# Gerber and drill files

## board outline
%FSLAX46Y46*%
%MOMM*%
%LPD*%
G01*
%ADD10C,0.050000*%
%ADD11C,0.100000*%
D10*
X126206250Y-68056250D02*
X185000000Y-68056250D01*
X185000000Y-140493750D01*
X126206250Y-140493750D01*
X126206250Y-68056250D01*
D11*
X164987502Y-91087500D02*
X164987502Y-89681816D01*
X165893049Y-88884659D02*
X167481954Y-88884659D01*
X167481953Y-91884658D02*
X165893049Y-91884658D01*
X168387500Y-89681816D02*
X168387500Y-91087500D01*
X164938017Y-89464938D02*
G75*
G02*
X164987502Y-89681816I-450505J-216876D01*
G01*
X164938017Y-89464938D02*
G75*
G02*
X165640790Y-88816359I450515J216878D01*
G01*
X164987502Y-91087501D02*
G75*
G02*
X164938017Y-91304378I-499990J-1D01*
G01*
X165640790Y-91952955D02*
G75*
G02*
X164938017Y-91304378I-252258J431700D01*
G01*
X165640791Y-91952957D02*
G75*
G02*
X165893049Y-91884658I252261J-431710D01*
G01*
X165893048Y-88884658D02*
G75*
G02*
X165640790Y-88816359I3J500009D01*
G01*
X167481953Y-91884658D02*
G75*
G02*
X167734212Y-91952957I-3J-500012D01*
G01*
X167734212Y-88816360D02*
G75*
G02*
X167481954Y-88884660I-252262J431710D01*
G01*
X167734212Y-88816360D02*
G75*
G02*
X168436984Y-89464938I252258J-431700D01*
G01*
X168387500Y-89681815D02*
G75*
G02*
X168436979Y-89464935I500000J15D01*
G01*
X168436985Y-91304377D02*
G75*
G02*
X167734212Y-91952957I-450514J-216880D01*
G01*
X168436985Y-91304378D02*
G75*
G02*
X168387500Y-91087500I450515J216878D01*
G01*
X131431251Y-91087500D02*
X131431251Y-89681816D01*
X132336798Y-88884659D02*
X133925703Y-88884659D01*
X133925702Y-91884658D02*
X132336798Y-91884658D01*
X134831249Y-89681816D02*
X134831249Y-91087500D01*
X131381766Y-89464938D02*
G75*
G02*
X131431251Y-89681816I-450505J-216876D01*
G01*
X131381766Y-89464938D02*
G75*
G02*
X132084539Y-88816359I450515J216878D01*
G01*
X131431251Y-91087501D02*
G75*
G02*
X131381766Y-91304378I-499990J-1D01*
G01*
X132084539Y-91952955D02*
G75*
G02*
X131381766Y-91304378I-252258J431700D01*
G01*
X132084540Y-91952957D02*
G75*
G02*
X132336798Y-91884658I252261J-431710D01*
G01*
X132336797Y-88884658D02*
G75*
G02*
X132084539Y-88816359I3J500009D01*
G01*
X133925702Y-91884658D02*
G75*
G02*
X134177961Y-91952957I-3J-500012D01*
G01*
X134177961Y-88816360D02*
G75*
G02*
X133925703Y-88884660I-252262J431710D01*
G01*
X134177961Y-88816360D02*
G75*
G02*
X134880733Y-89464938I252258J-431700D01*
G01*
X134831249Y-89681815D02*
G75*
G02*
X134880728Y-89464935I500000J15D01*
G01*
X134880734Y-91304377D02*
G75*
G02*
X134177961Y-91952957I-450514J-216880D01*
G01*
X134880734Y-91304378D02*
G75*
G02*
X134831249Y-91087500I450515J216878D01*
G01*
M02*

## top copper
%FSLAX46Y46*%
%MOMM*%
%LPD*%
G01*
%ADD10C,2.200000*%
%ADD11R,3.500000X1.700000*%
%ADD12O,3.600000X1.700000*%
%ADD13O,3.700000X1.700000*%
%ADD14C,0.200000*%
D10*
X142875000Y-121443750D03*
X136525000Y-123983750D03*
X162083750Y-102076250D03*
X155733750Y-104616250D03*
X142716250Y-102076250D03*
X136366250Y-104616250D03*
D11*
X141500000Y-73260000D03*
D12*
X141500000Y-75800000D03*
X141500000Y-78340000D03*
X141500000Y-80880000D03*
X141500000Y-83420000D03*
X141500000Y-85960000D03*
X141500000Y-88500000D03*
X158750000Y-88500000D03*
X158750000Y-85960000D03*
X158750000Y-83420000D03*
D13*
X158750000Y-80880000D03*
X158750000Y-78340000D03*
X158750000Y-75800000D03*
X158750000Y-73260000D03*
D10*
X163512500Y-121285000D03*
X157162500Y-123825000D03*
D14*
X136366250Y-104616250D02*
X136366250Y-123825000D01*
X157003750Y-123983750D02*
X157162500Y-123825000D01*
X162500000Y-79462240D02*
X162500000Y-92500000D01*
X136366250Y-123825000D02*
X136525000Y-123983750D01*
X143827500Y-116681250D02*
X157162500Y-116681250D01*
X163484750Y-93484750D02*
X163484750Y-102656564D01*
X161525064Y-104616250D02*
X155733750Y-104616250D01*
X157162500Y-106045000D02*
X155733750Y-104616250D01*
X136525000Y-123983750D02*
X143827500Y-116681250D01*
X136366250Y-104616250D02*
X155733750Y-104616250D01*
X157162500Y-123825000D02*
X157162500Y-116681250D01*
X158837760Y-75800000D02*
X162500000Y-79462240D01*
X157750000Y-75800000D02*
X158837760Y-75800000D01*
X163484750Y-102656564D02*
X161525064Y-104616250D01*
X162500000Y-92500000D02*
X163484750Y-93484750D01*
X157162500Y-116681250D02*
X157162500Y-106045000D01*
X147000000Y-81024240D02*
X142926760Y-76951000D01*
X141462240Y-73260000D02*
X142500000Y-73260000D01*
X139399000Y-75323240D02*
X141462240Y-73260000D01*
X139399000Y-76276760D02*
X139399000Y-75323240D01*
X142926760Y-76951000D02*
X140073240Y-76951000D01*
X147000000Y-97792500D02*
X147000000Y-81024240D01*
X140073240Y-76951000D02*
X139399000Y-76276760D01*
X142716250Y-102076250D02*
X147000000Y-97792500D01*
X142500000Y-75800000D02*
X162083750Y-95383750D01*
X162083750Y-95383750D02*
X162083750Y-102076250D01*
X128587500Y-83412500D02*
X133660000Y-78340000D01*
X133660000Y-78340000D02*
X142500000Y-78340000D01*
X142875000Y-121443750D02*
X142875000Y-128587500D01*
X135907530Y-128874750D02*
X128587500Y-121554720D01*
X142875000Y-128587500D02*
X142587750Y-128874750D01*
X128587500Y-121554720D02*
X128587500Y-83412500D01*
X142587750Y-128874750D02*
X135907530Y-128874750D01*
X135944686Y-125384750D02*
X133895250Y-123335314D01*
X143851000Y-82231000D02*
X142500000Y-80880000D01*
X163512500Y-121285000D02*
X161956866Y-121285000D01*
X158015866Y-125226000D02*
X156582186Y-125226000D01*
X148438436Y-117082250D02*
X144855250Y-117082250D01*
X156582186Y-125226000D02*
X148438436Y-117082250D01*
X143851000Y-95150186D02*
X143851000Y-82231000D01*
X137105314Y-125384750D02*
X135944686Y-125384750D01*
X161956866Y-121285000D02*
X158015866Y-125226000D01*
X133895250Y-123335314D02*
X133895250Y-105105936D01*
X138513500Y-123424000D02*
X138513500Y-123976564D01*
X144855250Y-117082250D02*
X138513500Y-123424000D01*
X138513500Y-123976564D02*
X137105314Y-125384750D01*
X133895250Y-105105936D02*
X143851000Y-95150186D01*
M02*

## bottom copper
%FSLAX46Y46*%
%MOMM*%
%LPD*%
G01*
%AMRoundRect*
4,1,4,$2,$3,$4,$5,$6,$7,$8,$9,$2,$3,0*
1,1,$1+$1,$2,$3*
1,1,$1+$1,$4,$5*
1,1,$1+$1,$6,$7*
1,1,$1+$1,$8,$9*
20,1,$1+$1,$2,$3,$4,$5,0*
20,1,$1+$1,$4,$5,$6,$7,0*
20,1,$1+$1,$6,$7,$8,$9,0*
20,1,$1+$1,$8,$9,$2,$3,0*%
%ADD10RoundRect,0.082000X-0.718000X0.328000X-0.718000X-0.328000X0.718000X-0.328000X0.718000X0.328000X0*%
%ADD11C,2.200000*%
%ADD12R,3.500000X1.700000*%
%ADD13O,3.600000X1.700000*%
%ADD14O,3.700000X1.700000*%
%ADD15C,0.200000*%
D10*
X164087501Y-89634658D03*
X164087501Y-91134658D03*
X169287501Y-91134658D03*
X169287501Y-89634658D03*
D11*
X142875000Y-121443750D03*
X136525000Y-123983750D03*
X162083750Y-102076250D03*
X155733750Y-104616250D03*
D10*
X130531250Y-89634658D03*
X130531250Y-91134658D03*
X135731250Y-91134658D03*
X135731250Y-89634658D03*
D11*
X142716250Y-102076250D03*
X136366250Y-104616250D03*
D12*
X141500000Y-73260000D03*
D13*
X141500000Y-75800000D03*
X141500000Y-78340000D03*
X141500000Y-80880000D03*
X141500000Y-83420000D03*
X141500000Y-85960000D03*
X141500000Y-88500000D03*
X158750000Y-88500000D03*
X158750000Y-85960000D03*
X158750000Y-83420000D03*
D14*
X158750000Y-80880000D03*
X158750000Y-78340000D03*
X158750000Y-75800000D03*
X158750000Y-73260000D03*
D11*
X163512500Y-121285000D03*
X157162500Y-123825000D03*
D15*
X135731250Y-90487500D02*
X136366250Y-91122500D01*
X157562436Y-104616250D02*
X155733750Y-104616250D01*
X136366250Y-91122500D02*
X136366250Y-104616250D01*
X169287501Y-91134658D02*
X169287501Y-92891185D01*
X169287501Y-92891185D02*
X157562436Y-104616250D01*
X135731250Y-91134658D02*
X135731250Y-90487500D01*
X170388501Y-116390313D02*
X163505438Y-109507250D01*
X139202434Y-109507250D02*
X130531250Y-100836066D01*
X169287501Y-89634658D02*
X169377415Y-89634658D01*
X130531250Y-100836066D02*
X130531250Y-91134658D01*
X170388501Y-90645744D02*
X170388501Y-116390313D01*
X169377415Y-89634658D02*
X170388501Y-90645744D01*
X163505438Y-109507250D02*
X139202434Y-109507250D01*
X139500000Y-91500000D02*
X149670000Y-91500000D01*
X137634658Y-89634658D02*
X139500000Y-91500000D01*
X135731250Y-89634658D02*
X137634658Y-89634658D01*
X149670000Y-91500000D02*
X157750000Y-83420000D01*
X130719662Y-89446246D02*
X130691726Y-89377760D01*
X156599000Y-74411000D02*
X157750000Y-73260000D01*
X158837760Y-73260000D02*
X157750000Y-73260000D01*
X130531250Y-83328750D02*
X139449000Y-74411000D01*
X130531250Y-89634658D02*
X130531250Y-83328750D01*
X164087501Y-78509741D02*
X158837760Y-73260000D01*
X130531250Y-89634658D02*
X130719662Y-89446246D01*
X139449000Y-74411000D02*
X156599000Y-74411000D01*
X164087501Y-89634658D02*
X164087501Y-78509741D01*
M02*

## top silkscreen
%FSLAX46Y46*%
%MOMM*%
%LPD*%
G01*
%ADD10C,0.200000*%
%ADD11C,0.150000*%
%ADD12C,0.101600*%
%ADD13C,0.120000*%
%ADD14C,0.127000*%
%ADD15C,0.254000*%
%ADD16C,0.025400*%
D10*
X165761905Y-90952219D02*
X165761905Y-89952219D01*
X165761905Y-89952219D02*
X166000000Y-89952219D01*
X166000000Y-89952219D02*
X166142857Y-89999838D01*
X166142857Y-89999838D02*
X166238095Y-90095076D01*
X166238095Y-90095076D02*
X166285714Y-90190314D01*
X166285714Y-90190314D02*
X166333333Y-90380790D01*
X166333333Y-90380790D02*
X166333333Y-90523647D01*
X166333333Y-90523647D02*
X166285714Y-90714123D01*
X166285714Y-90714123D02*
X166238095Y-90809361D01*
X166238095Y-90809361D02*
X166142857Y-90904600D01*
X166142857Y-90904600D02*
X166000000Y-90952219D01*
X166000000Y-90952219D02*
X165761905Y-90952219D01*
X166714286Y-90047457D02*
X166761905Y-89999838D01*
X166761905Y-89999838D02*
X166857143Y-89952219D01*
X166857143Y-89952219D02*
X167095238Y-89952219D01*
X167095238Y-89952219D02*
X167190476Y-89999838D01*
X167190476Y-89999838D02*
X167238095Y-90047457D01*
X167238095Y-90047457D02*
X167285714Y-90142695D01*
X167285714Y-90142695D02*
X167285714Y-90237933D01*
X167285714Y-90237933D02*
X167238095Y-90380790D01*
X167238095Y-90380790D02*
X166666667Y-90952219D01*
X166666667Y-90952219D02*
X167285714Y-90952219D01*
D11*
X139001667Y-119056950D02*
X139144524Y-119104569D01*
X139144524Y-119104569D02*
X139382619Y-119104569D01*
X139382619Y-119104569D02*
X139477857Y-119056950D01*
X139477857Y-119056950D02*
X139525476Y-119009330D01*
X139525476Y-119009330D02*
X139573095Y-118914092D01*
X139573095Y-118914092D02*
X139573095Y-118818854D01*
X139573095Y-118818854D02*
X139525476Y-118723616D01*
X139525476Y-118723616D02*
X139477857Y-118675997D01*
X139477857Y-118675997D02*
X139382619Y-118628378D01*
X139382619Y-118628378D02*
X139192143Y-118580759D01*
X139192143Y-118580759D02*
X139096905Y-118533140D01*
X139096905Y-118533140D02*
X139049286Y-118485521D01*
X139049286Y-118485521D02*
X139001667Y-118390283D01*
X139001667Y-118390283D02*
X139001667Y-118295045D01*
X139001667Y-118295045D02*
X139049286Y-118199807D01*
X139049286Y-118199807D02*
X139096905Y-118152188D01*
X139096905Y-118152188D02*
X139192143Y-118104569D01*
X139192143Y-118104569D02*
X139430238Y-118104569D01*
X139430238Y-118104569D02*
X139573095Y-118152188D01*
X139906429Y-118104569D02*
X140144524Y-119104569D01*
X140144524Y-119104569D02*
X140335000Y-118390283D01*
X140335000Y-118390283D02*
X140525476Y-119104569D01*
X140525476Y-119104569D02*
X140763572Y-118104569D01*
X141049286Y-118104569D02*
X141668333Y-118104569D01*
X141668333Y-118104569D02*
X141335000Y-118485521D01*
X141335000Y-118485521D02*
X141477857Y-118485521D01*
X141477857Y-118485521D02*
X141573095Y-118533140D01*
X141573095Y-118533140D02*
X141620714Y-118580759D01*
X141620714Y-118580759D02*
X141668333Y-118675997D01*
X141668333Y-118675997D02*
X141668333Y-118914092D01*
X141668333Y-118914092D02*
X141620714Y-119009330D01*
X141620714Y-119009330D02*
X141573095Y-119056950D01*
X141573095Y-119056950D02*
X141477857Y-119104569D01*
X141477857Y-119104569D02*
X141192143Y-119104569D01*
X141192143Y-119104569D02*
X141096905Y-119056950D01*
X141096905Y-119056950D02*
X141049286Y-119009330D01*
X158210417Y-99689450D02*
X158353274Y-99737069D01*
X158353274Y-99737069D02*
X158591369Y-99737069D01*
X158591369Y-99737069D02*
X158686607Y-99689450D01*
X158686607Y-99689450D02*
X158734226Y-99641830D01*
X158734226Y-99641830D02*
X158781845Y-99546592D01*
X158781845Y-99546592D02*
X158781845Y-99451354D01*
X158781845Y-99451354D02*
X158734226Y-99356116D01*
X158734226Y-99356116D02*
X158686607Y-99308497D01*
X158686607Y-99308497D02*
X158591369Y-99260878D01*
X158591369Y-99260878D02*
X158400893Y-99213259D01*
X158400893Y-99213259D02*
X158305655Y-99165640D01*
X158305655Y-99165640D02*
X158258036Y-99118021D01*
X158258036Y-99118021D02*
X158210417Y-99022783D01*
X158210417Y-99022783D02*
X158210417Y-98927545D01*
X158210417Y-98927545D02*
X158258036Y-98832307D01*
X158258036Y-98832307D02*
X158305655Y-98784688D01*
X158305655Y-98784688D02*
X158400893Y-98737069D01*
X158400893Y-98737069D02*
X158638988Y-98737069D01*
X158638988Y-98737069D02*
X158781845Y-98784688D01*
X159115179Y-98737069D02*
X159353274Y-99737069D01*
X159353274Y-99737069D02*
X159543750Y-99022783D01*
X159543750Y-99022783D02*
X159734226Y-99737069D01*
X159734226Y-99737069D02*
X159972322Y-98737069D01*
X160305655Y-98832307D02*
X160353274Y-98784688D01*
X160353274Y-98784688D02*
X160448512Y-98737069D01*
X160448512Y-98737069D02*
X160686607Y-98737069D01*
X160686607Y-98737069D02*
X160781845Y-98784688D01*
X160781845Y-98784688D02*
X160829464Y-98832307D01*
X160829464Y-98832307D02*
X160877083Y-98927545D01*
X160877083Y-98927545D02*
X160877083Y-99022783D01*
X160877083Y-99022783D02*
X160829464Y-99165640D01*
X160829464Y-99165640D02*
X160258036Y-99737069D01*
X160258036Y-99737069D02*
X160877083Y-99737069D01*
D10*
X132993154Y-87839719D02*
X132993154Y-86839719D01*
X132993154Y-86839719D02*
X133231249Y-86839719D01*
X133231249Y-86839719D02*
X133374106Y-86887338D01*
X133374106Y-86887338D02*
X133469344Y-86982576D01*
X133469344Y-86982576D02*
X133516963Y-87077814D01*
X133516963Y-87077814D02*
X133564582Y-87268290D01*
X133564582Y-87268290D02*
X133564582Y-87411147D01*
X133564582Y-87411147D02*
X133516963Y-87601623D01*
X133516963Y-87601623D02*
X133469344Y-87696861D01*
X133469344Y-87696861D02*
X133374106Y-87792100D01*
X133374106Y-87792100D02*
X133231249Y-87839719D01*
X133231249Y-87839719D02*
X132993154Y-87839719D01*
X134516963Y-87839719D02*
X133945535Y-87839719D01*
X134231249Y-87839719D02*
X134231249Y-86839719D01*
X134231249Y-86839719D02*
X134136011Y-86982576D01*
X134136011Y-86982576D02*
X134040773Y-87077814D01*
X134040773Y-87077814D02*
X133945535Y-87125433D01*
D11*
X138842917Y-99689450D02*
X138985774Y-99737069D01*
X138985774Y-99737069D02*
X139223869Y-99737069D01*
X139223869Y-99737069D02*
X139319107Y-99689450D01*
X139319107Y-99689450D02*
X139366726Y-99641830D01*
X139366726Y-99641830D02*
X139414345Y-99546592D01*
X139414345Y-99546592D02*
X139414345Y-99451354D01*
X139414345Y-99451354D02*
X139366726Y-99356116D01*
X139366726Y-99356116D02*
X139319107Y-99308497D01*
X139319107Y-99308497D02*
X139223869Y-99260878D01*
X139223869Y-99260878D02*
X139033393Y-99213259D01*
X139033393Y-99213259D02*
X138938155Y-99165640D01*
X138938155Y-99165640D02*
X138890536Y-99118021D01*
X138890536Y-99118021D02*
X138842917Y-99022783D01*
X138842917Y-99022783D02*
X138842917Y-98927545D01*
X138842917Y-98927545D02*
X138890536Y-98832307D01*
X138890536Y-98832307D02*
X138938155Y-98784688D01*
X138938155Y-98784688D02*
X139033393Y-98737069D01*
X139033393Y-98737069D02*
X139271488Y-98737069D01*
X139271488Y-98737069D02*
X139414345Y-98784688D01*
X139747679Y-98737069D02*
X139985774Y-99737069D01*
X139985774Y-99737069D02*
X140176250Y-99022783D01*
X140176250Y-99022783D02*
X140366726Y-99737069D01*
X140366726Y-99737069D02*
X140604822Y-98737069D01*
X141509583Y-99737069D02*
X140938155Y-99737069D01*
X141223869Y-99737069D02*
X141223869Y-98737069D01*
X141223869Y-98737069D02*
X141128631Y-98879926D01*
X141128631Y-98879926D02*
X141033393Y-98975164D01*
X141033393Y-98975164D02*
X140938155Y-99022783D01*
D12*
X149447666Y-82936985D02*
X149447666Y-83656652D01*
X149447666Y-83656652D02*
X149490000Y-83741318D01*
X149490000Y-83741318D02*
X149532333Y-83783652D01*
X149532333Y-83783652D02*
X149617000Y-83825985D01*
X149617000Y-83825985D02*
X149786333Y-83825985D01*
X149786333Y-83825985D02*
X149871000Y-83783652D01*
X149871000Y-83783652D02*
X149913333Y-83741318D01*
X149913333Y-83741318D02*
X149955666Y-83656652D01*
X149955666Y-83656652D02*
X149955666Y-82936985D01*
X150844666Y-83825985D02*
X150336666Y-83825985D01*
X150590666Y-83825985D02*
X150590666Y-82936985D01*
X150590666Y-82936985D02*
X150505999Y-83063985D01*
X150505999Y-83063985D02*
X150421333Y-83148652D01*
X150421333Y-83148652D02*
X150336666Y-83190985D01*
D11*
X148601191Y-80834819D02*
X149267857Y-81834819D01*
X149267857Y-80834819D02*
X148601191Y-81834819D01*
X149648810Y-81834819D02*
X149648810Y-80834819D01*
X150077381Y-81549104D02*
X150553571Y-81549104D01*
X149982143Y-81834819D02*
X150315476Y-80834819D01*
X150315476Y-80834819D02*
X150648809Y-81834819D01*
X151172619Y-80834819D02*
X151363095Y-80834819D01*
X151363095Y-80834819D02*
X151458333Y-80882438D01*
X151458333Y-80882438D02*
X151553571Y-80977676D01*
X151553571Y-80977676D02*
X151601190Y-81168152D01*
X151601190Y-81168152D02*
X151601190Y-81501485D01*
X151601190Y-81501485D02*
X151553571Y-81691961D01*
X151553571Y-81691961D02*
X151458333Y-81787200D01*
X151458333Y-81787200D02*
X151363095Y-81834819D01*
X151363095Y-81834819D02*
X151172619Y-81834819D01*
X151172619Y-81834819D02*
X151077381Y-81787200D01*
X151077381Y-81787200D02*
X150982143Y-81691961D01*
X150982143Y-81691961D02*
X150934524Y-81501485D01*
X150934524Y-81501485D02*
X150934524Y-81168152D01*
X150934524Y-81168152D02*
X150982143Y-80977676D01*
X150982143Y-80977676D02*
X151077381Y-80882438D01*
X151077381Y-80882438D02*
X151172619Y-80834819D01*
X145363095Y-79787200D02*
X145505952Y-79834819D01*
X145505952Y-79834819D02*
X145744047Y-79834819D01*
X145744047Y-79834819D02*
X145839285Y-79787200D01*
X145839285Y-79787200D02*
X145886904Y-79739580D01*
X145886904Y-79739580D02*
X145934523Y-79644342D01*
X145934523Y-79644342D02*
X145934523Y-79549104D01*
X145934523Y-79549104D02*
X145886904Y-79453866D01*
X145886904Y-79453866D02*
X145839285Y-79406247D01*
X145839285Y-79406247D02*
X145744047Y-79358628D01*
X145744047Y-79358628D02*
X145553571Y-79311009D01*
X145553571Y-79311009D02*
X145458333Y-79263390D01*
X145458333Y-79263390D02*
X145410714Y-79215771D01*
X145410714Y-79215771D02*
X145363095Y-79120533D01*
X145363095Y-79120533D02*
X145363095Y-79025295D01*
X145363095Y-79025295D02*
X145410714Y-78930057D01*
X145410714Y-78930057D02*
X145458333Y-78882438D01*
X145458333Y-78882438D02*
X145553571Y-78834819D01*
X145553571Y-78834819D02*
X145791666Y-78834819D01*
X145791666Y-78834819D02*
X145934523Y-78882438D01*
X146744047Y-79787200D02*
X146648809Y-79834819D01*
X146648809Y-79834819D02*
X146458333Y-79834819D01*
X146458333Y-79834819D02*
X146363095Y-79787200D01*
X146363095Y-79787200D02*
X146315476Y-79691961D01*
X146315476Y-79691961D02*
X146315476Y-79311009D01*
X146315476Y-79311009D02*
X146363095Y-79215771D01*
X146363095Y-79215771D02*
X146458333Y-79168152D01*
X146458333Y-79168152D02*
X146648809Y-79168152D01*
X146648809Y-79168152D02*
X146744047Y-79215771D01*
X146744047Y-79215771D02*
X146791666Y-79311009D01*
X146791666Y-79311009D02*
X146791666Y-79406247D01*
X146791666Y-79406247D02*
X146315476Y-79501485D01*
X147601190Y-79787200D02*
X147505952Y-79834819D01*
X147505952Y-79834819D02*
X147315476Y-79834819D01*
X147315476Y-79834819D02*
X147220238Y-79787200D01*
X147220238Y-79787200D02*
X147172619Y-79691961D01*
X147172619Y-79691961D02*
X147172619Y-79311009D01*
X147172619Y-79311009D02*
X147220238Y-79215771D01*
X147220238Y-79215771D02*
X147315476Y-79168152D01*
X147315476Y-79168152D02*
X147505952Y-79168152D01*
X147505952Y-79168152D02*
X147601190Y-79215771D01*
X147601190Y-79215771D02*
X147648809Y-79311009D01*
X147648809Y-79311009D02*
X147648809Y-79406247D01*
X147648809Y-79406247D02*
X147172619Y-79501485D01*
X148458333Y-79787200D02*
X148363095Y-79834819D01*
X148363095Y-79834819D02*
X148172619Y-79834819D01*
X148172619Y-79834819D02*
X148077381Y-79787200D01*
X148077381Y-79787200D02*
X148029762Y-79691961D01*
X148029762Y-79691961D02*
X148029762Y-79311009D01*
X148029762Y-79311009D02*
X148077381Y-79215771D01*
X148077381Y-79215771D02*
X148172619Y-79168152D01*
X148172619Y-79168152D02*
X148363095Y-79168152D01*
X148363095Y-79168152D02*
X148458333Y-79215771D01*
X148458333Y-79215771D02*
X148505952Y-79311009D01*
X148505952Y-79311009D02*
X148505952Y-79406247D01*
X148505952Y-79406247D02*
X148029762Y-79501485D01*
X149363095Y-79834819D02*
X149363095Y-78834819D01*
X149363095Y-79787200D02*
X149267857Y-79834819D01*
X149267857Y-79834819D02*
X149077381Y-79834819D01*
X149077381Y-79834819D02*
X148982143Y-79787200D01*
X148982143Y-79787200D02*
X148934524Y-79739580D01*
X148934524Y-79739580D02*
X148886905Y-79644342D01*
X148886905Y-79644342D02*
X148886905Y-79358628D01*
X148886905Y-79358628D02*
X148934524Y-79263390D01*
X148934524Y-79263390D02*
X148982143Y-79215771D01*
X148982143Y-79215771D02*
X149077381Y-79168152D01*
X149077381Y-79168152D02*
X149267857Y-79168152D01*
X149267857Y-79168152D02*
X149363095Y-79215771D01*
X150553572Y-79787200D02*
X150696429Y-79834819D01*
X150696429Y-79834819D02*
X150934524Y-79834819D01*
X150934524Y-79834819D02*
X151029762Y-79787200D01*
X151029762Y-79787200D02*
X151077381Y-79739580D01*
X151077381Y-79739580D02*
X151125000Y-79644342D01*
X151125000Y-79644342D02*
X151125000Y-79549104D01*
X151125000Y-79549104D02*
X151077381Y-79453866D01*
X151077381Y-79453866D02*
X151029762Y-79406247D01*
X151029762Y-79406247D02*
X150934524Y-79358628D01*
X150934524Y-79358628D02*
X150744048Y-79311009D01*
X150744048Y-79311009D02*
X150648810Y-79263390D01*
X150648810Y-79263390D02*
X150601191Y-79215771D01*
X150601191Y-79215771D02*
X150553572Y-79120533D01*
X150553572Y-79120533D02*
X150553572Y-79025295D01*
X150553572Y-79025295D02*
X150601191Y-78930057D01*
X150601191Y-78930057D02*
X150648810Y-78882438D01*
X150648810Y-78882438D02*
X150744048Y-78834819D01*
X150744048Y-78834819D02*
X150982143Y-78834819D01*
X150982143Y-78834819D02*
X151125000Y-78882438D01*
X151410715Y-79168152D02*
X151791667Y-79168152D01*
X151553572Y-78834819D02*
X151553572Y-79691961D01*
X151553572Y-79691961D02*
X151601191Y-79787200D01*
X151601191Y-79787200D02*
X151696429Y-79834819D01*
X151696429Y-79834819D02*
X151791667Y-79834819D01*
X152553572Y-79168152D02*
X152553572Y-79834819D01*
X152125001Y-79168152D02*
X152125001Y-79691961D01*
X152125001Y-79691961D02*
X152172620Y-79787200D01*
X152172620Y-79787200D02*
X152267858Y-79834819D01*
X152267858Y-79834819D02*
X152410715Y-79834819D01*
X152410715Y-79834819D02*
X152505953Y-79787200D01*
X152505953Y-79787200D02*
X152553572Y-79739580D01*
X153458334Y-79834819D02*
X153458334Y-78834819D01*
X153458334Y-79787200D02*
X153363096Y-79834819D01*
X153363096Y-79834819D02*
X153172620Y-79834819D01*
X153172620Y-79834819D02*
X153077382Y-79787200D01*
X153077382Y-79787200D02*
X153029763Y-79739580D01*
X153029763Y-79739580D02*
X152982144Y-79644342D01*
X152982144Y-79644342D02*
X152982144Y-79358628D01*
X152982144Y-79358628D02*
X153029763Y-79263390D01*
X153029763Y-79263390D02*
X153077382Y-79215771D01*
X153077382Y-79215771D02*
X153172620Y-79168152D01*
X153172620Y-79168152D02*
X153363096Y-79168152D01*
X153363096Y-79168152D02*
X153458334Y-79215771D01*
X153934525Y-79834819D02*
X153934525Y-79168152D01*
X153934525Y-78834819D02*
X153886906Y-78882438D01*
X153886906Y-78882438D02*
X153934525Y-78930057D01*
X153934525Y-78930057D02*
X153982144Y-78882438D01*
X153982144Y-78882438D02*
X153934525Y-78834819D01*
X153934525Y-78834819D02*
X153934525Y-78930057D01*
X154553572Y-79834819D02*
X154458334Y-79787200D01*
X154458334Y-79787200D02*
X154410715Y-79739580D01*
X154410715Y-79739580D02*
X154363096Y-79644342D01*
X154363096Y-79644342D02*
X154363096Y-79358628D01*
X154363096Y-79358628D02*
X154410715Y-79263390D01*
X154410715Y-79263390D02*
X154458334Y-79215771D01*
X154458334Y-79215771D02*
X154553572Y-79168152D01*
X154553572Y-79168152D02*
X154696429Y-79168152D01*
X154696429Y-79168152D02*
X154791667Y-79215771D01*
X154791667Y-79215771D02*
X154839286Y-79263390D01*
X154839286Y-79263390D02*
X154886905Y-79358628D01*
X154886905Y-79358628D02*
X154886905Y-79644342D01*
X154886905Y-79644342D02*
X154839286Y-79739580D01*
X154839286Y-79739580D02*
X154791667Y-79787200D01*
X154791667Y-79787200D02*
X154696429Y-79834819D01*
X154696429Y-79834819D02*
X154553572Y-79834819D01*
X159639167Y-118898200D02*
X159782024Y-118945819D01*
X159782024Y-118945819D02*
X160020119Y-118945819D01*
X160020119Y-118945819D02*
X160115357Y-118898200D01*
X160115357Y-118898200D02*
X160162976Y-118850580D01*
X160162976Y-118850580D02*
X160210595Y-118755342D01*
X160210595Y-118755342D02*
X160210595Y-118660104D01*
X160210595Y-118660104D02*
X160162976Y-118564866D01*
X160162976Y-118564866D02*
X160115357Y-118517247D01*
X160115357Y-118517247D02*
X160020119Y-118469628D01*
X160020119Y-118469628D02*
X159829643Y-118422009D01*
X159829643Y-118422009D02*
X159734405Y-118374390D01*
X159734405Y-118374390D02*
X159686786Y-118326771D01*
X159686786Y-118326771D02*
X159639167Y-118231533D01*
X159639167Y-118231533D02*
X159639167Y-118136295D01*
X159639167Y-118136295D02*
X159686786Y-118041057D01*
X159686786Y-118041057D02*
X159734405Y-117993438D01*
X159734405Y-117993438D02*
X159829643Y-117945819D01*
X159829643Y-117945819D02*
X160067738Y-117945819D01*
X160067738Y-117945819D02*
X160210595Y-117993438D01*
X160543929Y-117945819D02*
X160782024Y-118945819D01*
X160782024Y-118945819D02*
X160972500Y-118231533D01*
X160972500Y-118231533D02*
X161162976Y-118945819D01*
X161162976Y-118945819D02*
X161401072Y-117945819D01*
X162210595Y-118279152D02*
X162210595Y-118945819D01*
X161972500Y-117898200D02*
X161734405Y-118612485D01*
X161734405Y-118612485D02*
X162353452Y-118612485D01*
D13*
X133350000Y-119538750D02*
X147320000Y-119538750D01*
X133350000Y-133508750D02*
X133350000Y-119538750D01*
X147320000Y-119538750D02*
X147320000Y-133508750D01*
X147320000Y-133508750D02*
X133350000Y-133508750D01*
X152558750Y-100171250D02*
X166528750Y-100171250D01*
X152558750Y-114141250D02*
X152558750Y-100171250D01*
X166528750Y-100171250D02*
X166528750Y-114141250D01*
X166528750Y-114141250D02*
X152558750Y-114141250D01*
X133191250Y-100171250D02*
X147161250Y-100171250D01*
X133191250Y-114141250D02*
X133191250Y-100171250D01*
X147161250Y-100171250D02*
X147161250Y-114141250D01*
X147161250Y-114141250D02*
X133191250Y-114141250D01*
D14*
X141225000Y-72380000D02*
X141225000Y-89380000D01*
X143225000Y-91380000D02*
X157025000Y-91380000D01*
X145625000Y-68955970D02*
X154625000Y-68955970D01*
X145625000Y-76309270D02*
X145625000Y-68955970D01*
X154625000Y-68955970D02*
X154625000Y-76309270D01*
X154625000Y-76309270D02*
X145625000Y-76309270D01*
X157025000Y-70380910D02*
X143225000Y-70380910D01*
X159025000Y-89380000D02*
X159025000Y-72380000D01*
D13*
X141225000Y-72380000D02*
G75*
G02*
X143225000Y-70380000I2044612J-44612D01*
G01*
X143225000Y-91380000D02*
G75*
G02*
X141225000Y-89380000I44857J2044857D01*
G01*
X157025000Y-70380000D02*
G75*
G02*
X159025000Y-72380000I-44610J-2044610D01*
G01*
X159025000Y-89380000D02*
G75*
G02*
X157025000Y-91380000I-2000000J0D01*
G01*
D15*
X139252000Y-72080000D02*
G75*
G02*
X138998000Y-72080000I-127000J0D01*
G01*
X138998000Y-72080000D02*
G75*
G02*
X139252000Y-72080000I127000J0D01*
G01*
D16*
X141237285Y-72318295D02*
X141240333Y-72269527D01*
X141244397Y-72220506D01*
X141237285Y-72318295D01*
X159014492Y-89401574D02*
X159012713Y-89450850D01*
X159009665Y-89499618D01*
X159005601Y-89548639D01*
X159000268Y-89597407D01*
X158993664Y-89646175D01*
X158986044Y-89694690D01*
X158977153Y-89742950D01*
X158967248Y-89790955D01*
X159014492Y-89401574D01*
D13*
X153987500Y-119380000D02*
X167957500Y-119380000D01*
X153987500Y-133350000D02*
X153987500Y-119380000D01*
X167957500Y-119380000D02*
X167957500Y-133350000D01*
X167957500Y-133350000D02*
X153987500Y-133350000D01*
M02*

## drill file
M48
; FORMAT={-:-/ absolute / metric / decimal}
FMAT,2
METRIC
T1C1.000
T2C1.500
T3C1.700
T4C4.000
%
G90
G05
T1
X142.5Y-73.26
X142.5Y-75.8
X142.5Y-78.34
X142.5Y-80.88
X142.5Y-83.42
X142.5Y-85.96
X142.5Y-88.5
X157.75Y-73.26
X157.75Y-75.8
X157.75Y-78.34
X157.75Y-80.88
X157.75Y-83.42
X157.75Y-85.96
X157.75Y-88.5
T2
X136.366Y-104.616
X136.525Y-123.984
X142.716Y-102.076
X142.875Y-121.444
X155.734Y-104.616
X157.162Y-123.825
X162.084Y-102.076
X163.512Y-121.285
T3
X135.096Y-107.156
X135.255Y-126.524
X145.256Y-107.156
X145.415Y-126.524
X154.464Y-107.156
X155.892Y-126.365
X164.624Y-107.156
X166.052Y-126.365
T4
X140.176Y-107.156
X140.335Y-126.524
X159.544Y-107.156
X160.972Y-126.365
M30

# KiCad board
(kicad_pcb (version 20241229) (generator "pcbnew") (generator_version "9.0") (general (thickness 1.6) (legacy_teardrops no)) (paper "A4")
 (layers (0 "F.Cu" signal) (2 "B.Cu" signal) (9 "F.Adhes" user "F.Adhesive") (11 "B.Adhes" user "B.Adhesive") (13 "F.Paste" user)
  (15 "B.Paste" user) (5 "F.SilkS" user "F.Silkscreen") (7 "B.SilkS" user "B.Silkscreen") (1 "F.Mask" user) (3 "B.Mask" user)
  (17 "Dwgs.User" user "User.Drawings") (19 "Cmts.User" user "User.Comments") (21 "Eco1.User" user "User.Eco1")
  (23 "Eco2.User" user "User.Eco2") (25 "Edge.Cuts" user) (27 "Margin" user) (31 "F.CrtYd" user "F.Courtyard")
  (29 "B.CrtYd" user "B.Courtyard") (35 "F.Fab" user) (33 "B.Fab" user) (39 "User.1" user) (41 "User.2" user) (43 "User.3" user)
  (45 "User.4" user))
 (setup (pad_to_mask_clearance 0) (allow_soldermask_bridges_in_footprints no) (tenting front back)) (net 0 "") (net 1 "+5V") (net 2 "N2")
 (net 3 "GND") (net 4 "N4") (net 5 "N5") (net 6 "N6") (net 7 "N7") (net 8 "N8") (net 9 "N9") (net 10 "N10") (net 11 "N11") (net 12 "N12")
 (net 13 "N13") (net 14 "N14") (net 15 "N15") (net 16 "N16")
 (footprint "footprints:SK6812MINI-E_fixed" (layer "F.Cu") (at 166.6875 90.4875)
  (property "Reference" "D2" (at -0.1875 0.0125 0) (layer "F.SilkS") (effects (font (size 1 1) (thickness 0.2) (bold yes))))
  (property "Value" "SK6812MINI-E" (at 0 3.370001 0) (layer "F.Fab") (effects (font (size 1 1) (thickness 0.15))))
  (fp_line (start -1.699998 0.6) (end -1.699998 -0.805684) (stroke (width 0.1) (type solid)) (layer "Edge.Cuts"))
  (fp_line (start -0.794451 -1.602841) (end 0.794454 -1.602841) (stroke (width 0.1) (type solid)) (layer "Edge.Cuts"))
  (fp_line (start 0.794453 1.397158) (end -0.794451 1.397158) (stroke (width 0.1) (type solid)) (layer "Edge.Cuts"))
  (fp_line (start 1.7 -0.805684) (end 1.7 0.6) (stroke (width 0.1) (type solid)) (layer "Edge.Cuts"))
  (fp_arc (start -1.749483 -1.022562) (mid -1.712526 -0.91691) (end -1.699998 -0.805684) (stroke (width 0.1) (type solid))
   (layer "Edge.Cuts"))
  (fp_arc (start -1.749483 -1.022562) (mid -1.63807 -1.606877) (end -1.04671 -1.671141) (stroke (width 0.1) (type solid))
   (layer "Edge.Cuts"))
  (fp_arc (start -1.699998 0.600001) (mid -1.712526 0.711226) (end -1.749483 0.816878) (stroke (width 0.1) (type solid)) (layer "Edge.Cuts"))
  (fp_arc (start -1.04671 1.465455) (mid -1.638069 1.401192) (end -1.749483 0.816878) (stroke (width 0.1) (type solid)) (layer "Edge.Cuts"))
  (fp_arc (start -1.046709 1.465457) (mid -0.925121 1.414535) (end -0.794451 1.397158) (stroke (width 0.1) (type solid)) (layer "Edge.Cuts"))
  (fp_arc (start -0.794452 -1.602842) (mid -0.925122 -1.620219) (end -1.04671 -1.671141) (stroke (width 0.1) (type solid))
   (layer "Edge.Cuts"))
  (fp_arc (start 0.794453 1.397158) (mid 0.925124 1.414535) (end 1.046712 1.465457) (stroke (width 0.1) (type solid)) (layer "Edge.Cuts"))
  (fp_arc (start 1.046712 -1.67114) (mid 0.925124 -1.620218) (end 0.794454 -1.602841) (stroke (width 0.1) (type solid)) (layer "Edge.Cuts"))
  (fp_arc (start 1.046712 -1.67114) (mid 1.638072 -1.606876) (end 1.749485 -1.022562) (stroke (width 0.1) (type solid)) (layer "Edge.Cuts"))
  (fp_arc (start 1.7 -0.805685) (mid 1.712528 -0.91691) (end 1.749485 -1.022562) (stroke (width 0.1) (type solid)) (layer "Edge.Cuts"))
  (fp_arc (start 1.749485 0.816877) (mid 1.638073 1.401193) (end 1.046712 1.465457) (stroke (width 0.1) (type solid)) (layer "Edge.Cuts"))
  (fp_arc (start 1.749485 0.816878) (mid 1.712528 0.711226) (end 1.7 0.6) (stroke (width 0.1) (type solid)) (layer "Edge.Cuts"))
  (pad "1" smd roundrect (at -2.599999 -0.852842 270) (size 0.82 1.6) (layers "B.Cu" "B.Mask" "B.Paste") (roundrect_rratio 0.1)
   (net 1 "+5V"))
  (pad "2" smd roundrect (at -2.599999 0.647158 270) (size 0.82 1.6) (layers "B.Cu" "B.Mask" "B.Paste") (roundrect_rratio 0.1) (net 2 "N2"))
  (pad "3" smd roundrect (at 2.600001 0.647158 270) (size 0.82 1.6) (layers "B.Cu" "B.Mask" "B.Paste") (roundrect_rratio 0.1) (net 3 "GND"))
  (pad "4" smd roundrect (at 2.600001 -0.852842 270) (size 0.82 1.6) (layers "B.Cu" "B.Mask" "B.Paste") (roundrect_rratio 0.1) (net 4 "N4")))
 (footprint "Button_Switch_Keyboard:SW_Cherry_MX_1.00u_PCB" (layer "F.Cu") (at 142.82 117.03875)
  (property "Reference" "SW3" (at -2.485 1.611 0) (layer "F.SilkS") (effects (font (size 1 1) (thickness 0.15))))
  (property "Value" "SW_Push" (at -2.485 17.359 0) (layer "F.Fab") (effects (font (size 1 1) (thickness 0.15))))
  (fp_line (start -9.47 2.5) (end 4.5 2.5) (stroke (width 0.12) (type solid)) (layer "F.SilkS"))
  (fp_line (start -9.47 16.47) (end -9.47 2.5) (stroke (width 0.12) (type solid)) (layer "F.SilkS"))
  (fp_line (start 4.5 2.5) (end 4.5 16.47) (stroke (width 0.12) (type solid)) (layer "F.SilkS"))
  (fp_line (start 4.5 16.47) (end -9.47 16.47) (stroke (width 0.12) (type solid)) (layer "F.SilkS"))
  (pad "" np_thru_hole circle (at -7.565 9.485) (size 1.7 1.7) (drill 1.7) (layers "*.Cu" "*.Mask"))
  (pad "" np_thru_hole circle (at -2.485 9.485) (size 4 4) (drill 4) (layers "*.Cu" "*.Mask"))
  (pad "" np_thru_hole circle (at 2.595 9.485) (size 1.7 1.7) (drill 1.7) (layers "*.Cu" "*.Mask"))
  (pad "1" thru_hole circle (at 0.055 4.405) (size 2.2 2.2) (drill 1.5) (layers "*.Cu" "*.Mask") (remove_unused_layers no) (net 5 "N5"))
  (pad "2" thru_hole circle (at -6.295 6.945) (size 2.2 2.2) (drill 1.5) (layers "*.Cu" "*.Mask") (remove_unused_layers no) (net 3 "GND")))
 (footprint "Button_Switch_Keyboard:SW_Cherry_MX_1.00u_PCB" (layer "F.Cu") (at 162.02875 97.67125)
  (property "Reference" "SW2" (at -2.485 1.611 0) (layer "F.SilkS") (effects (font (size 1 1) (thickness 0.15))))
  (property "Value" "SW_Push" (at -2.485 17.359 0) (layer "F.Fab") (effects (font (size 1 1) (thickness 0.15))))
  (fp_line (start -9.47 2.5) (end 4.5 2.5) (stroke (width 0.12) (type solid)) (layer "F.SilkS"))
  (fp_line (start -9.47 16.47) (end -9.47 2.5) (stroke (width 0.12) (type solid)) (layer "F.SilkS"))
  (fp_line (start 4.5 2.5) (end 4.5 16.47) (stroke (width 0.12) (type solid)) (layer "F.SilkS"))
  (fp_line (start 4.5 16.47) (end -9.47 16.47) (stroke (width 0.12) (type solid)) (layer "F.SilkS"))
  (pad "" np_thru_hole circle (at -7.565 9.485) (size 1.7 1.7) (drill 1.7) (layers "*.Cu" "*.Mask"))
  (pad "" np_thru_hole circle (at -2.485 9.485) (size 4 4) (drill 4) (layers "*.Cu" "*.Mask"))
  (pad "" np_thru_hole circle (at 2.595 9.485) (size 1.7 1.7) (drill 1.7) (layers "*.Cu" "*.Mask"))
  (pad "1" thru_hole circle (at 0.055 4.405) (size 2.2 2.2) (drill 1.5) (layers "*.Cu" "*.Mask") (remove_unused_layers no) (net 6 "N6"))
  (pad "2" thru_hole circle (at -6.295 6.945) (size 2.2 2.2) (drill 1.5) (layers "*.Cu" "*.Mask") (remove_unused_layers no) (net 3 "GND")))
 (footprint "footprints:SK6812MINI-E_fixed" (layer "F.Cu") (at 133.131249 90.4875)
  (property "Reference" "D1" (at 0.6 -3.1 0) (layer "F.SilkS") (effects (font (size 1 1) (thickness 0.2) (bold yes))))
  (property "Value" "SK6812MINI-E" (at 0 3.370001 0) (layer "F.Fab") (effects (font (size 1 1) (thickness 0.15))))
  (fp_line (start -1.699998 0.6) (end -1.699998 -0.805684) (stroke (width 0.1) (type solid)) (layer "Edge.Cuts"))
  (fp_line (start -0.794451 -1.602841) (end 0.794454 -1.602841) (stroke (width 0.1) (type solid)) (layer "Edge.Cuts"))
  (fp_line (start 0.794453 1.397158) (end -0.794451 1.397158) (stroke (width 0.1) (type solid)) (layer "Edge.Cuts"))
  (fp_line (start 1.7 -0.805684) (end 1.7 0.6) (stroke (width 0.1) (type solid)) (layer "Edge.Cuts"))
  (fp_arc (start -1.749483 -1.022562) (mid -1.712526 -0.91691) (end -1.699998 -0.805684) (stroke (width 0.1) (type solid))
   (layer "Edge.Cuts"))
  (fp_arc (start -1.749483 -1.022562) (mid -1.63807 -1.606877) (end -1.04671 -1.671141) (stroke (width 0.1) (type solid))
   (layer "Edge.Cuts"))
  (fp_arc (start -1.699998 0.600001) (mid -1.712526 0.711226) (end -1.749483 0.816878) (stroke (width 0.1) (type solid)) (layer "Edge.Cuts"))
  (fp_arc (start -1.04671 1.465455) (mid -1.638069 1.401192) (end -1.749483 0.816878) (stroke (width 0.1) (type solid)) (layer "Edge.Cuts"))
  (fp_arc (start -1.046709 1.465457) (mid -0.925121 1.414535) (end -0.794451 1.397158) (stroke (width 0.1) (type solid)) (layer "Edge.Cuts"))
  (fp_arc (start -0.794452 -1.602842) (mid -0.925122 -1.620219) (end -1.04671 -1.671141) (stroke (width 0.1) (type solid))
   (layer "Edge.Cuts"))
  (fp_arc (start 0.794453 1.397158) (mid 0.925124 1.414535) (end 1.046712 1.465457) (stroke (width 0.1) (type solid)) (layer "Edge.Cuts"))
  (fp_arc (start 1.046712 -1.67114) (mid 0.925124 -1.620218) (end 0.794454 -1.602841) (stroke (width 0.1) (type solid)) (layer "Edge.Cuts"))
  (fp_arc (start 1.046712 -1.67114) (mid 1.638072 -1.606876) (end 1.749485 -1.022562) (stroke (width 0.1) (type solid)) (layer "Edge.Cuts"))
  (fp_arc (start 1.7 -0.805685) (mid 1.712528 -0.91691) (end 1.749485 -1.022562) (stroke (width 0.1) (type solid)) (layer "Edge.Cuts"))
  (fp_arc (start 1.749485 0.816877) (mid 1.638073 1.401193) (end 1.046712 1.465457) (stroke (width 0.1) (type solid)) (layer "Edge.Cuts"))
  (fp_arc (start 1.749485 0.816878) (mid 1.712528 0.711226) (end 1.7 0.6) (stroke (width 0.1) (type solid)) (layer "Edge.Cuts"))
  (pad "1" smd roundrect (at -2.599999 -0.852842 270) (size 0.82 1.6) (layers "B.Cu" "B.Mask" "B.Paste") (roundrect_rratio 0.1)
   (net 1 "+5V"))
  (pad "2" smd roundrect (at -2.599999 0.647158 270) (size 0.82 1.6) (layers "B.Cu" "B.Mask" "B.Paste") (roundrect_rratio 0.1) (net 4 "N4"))
  (pad "3" smd roundrect (at 2.600001 0.647158 270) (size 0.82 1.6) (layers "B.Cu" "B.Mask" "B.Paste") (roundrect_rratio 0.1) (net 3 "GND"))
  (pad "4" smd roundrect (at 2.600001 -0.852842 270) (size 0.82 1.6) (layers "B.Cu" "B.Mask" "B.Paste") (roundrect_rratio 0.1) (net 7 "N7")))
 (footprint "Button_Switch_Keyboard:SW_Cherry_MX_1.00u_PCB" (layer "F.Cu") (at 142.66125 97.67125)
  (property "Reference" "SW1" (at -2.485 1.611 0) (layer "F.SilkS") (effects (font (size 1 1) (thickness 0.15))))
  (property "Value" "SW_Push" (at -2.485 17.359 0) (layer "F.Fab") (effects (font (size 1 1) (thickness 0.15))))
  (fp_line (start -9.47 2.5) (end 4.5 2.5) (stroke (width 0.12) (type solid)) (layer "F.SilkS"))
  (fp_line (start -9.47 16.47) (end -9.47 2.5) (stroke (width 0.12) (type solid)) (layer "F.SilkS"))
  (fp_line (start 4.5 2.5) (end 4.5 16.47) (stroke (width 0.12) (type solid)) (layer "F.SilkS"))
  (fp_line (start 4.5 16.47) (end -9.47 16.47) (stroke (width 0.12) (type solid)) (layer "F.SilkS"))
  (pad "" np_thru_hole circle (at -7.565 9.485) (size 1.7 1.7) (drill 1.7) (layers "*.Cu" "*.Mask"))
  (pad "" np_thru_hole circle (at -2.485 9.485) (size 4 4) (drill 4) (layers "*.Cu" "*.Mask"))
  (pad "" np_thru_hole circle (at 2.595 9.485) (size 1.7 1.7) (drill 1.7) (layers "*.Cu" "*.Mask"))
  (pad "1" thru_hole circle (at 0.055 4.405) (size 2.2 2.2) (drill 1.5) (layers "*.Cu" "*.Mask") (remove_unused_layers no) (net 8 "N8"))
  (pad "2" thru_hole circle (at -6.295 6.945) (size 2.2 2.2) (drill 1.5) (layers "*.Cu" "*.Mask") (remove_unused_layers no) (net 3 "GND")))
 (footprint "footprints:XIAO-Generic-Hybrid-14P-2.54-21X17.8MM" (layer "F.Cu") (at 150.125 80.88)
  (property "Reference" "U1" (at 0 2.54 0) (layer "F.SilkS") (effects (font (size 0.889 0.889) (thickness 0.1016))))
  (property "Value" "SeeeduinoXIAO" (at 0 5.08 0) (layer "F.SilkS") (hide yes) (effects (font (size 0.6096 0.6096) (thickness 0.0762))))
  (fp_line (start -8.9 -8.5) (end -8.9 8.5) (stroke (width 0.127) (type solid)) (layer "F.SilkS"))
  (fp_line (start -6.9 10.5) (end 6.9 10.5) (stroke (width 0.127) (type solid)) (layer "F.SilkS"))
  (fp_line (start -4.5 -11.92403) (end 4.5 -11.92403) (stroke (width 0.127) (type solid)) (layer "F.SilkS"))
  (fp_line (start -4.5 -4.57073) (end -4.5 -11.92403) (stroke (width 0.127) (type solid)) (layer "F.SilkS"))
  (fp_line (start 4.5 -11.92403) (end 4.5 -4.57073) (stroke (width 0.127) (type solid)) (layer "F.SilkS"))
  (fp_line (start 4.5 -4.57073) (end -4.5 -4.57073) (stroke (width 0.127) (type solid)) (layer "F.SilkS"))
  (fp_line (start 6.9 -10.49909) (end -6.9 -10.49909) (stroke (width 0.127) (type solid)) (layer "F.SilkS"))
  (fp_line (start 8.9 8.5) (end 8.9 -8.5) (stroke (width 0.127) (type solid)) (layer "F.SilkS"))
  (fp_arc (start -8.9 -8.5) (mid -8.301491 -9.901491) (end -6.9 -10.5) (stroke (width 0.12) (type solid)) (layer "F.SilkS"))
  (fp_arc (start -6.9 10.5) (mid -8.301423 9.901423) (end -8.9 8.5) (stroke (width 0.12) (type solid)) (layer "F.SilkS"))
  (fp_arc (start 6.9 -10.5) (mid 8.301491 -9.901491) (end 8.9 -8.5) (stroke (width 0.12) (type solid)) (layer "F.SilkS"))
  (fp_arc (start 8.9 8.5) (mid 8.314214 9.914214) (end 6.9 10.5) (stroke (width 0.12) (type solid)) (layer "F.SilkS"))
  (fp_circle (center -11 -8.8) (end -11 -9.054) (stroke (width 0) (type solid)) (fill yes) (layer "F.SilkS"))
  (fp_poly
   (pts (xy -8.887715 -8.561705) (xy -8.884667 -8.610473) (xy -8.880603 -8.659494)) (stroke (width 0.0254) (type solid)) (fill no)
   (layer "F.SilkS"))
  (fp_poly
   (pts (xy 8.889492 8.521574) (xy 8.887713 8.57085) (xy 8.884665 8.619618) (xy 8.880601 8.668639) (xy 8.875268 8.717407)
    (xy 8.868664 8.766175) (xy 8.861044 8.81469) (xy 8.852153 8.86295) (xy 8.842248 8.910955))
   (stroke (width 0.0254) (type solid)) (fill no) (layer "F.SilkS"))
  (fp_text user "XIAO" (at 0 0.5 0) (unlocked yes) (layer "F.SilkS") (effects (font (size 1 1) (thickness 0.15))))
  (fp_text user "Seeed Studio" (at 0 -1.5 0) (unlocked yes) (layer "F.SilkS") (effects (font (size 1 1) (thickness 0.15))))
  (pad "1" thru_hole rect (at -7.625 -7.62) (size 3.5 1.7) (drill 1 (offset -1 0)) (layers "*.Cu" "*.Mask") (remove_unused_layers no)
   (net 8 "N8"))
  (pad "2" thru_hole oval (at -7.625 -5.08) (size 3.6 1.7) (drill 1 (offset -1 0)) (layers "*.Cu" "*.Mask") (remove_unused_layers no)
   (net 6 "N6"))
  (pad "3" thru_hole oval (at -7.625 -2.54) (size 3.6 1.7) (drill 1 (offset -1 0)) (layers "*.Cu" "*.Mask") (remove_unused_layers no)
   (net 5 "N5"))
  (pad "4" thru_hole oval (at -7.625 0) (size 3.6 1.7) (drill 1 (offset -1 0)) (layers "*.Cu" "*.Mask") (remove_unused_layers no)
   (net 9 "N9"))
  (pad "5" thru_hole oval (at -7.625 2.54) (size 3.6 1.7) (drill 1 (offset -1 0)) (layers "*.Cu" "*.Mask") (remove_unused_layers no)
   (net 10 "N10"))
  (pad "6" thru_hole oval (at -7.625 5.08 180) (size 3.6 1.7) (drill 1 (offset 1 0)) (layers "*.Cu" "*.Mask") (remove_unused_layers no)
   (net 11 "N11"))
  (pad "7" thru_hole oval (at -7.625 7.62) (size 3.6 1.7) (drill 1 (offset -1 0)) (layers "*.Cu" "*.Mask") (remove_unused_layers no)
   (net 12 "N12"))
  (pad "8" thru_hole oval (at 7.625 7.62) (size 3.6 1.7) (drill 1 (offset 1 0)) (layers "*.Cu" "*.Mask") (remove_unused_layers no)
   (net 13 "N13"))
  (pad "9" thru_hole oval (at 7.625 5.08) (size 3.6 1.7) (drill 1 (offset 1 0)) (layers "*.Cu" "*.Mask") (remove_unused_layers no)
   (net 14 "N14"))
  (pad "10" thru_hole oval (at 7.625 2.54) (size 3.6 1.7) (drill 1 (offset 1 0)) (layers "*.Cu" "*.Mask") (remove_unused_layers no)
   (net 7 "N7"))
  (pad "11" thru_hole oval (at 7.625 0) (size 3.7 1.7) (drill 1 (offset 1 0)) (layers "*.Cu" "*.Mask") (remove_unused_layers no)
   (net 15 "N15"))
  (pad "12" thru_hole oval (at 7.625 -2.54) (size 3.7 1.7) (drill 1 (offset 1 0)) (layers "*.Cu" "*.Mask") (remove_unused_layers no)
   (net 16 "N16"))
  (pad "13" thru_hole oval (at 7.625 -5.08) (size 3.7 1.7) (drill 1 (offset 1 0)) (layers "*.Cu" "*.Mask") (remove_unused_layers no)
   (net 3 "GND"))
  (pad "14" thru_hole oval (at 7.625 -7.62) (size 3.7 1.7) (drill 1 (offset 1 0)) (layers "*.Cu" "*.Mask") (remove_unused_layers no)
   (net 1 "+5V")))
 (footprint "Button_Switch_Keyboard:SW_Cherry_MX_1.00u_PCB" (layer "F.Cu") (at 163.4575 116.88)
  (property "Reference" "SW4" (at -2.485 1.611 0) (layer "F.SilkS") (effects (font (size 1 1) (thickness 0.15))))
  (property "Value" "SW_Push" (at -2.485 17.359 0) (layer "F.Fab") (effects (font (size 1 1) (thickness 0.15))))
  (fp_line (start -9.47 2.5) (end 4.5 2.5) (stroke (width 0.12) (type solid)) (layer "F.SilkS"))
  (fp_line (start -9.47 16.47) (end -9.47 2.5) (stroke (width 0.12) (type solid)) (layer "F.SilkS"))
  (fp_line (start 4.5 2.5) (end 4.5 16.47) (stroke (width 0.12) (type solid)) (layer "F.SilkS"))
  (fp_line (start 4.5 16.47) (end -9.47 16.47) (stroke (width 0.12) (type solid)) (layer "F.SilkS"))
  (pad "" np_thru_hole circle (at -7.565 9.485) (size 1.7 1.7) (drill 1.7) (layers "*.Cu" "*.Mask"))
  (pad "" np_thru_hole circle (at -2.485 9.485) (size 4 4) (drill 4) (layers "*.Cu" "*.Mask"))
  (pad "" np_thru_hole circle (at 2.595 9.485) (size 1.7 1.7) (drill 1.7) (layers "*.Cu" "*.Mask"))
  (pad "1" thru_hole circle (at 0.055 4.405) (size 2.2 2.2) (drill 1.5) (layers "*.Cu" "*.Mask") (remove_unused_layers no) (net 9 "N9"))
  (pad "2" thru_hole circle (at -6.295 6.945) (size 2.2 2.2) (drill 1.5) (layers "*.Cu" "*.Mask") (remove_unused_layers no) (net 3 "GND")))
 (gr_rect (start 126.20625 68.05625) (end 185 140.49375) (stroke (width 0.05) (type solid)) (fill no) (layer "Edge.Cuts"))
 (segment (start 136.36625 104.61625) (end 136.36625 123.825) (width 0.2) (layer "F.Cu") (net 3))
 (segment (start 157.00375 123.98375) (end 157.1625 123.825) (width 0.2) (layer "F.Cu") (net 3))
 (segment (start 162.5 79.46224) (end 162.5 92.5) (width 0.2) (layer "F.Cu") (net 3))
 (segment (start 136.36625 123.825) (end 136.525 123.98375) (width 0.2) (layer "F.Cu") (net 3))
 (segment (start 143.8275 116.68125) (end 157.1625 116.68125) (width 0.2) (layer "F.Cu") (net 3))
 (segment (start 163.48475 93.48475) (end 163.48475 102.656564) (width 0.2) (layer "F.Cu") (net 3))
 (segment (start 161.525064 104.61625) (end 155.73375 104.61625) (width 0.2) (layer "F.Cu") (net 3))
 (segment (start 157.1625 106.045) (end 155.73375 104.61625) (width 0.2) (layer "F.Cu") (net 3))
 (segment (start 136.525 123.98375) (end 143.8275 116.68125) (width 0.2) (layer "F.Cu") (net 3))
 (segment (start 136.36625 104.61625) (end 155.73375 104.61625) (width 0.2) (layer "F.Cu") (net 3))
 (segment (start 157.1625 123.825) (end 157.1625 116.68125) (width 0.2) (layer "F.Cu") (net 3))
 (segment (start 158.83776 75.8) (end 162.5 79.46224) (width 0.2) (layer "F.Cu") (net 3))
 (segment (start 157.75 75.8) (end 158.83776 75.8) (width 0.2) (layer "F.Cu") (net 3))
 (segment (start 163.48475 102.656564) (end 161.525064 104.61625) (width 0.2) (layer "F.Cu") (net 3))
 (segment (start 162.5 92.5) (end 163.48475 93.48475) (width 0.2) (layer "F.Cu") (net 3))
 (segment (start 157.1625 116.68125) (end 157.1625 106.045) (width 0.2) (layer "F.Cu") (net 3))
 (segment (start 135.73125 90.4875) (end 136.36625 91.1225) (width 0.2) (layer "B.Cu") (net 3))
 (segment (start 157.562436 104.61625) (end 155.73375 104.61625) (width 0.2) (layer "B.Cu") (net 3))
 (segment (start 136.36625 91.1225) (end 136.36625 104.61625) (width 0.2) (layer "B.Cu") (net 3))
 (segment (start 169.287501 91.134658) (end 169.287501 92.891185) (width 0.2) (layer "B.Cu") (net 3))
 (segment (start 169.287501 92.891185) (end 157.562436 104.61625) (width 0.2) (layer "B.Cu") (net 3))
 (segment (start 135.73125 91.134658) (end 135.73125 90.4875) (width 0.2) (layer "B.Cu") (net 3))
 (segment (start 170.388501 116.390313) (end 163.505438 109.50725) (width 0.2) (layer "B.Cu") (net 4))
 (segment (start 139.202434 109.50725) (end 130.53125 100.836066) (width 0.2) (layer "B.Cu") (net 4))
 (segment (start 169.287501 89.634658) (end 169.377415 89.634658) (width 0.2) (layer "B.Cu") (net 4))
 (segment (start 130.53125 100.836066) (end 130.53125 91.134658) (width 0.2) (layer "B.Cu") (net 4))
 (segment (start 170.388501 90.645744) (end 170.388501 116.390313) (width 0.2) (layer "B.Cu") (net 4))
 (segment (start 169.377415 89.634658) (end 170.388501 90.645744) (width 0.2) (layer "B.Cu") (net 4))
 (segment (start 163.505438 109.50725) (end 139.202434 109.50725) (width 0.2) (layer "B.Cu") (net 4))
 (segment (start 139.5 91.5) (end 149.67 91.5) (width 0.2) (layer "B.Cu") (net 7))
 (segment (start 137.634658 89.634658) (end 139.5 91.5) (width 0.2) (layer "B.Cu") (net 7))
 (segment (start 135.73125 89.634658) (end 137.634658 89.634658) (width 0.2) (layer "B.Cu") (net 7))
 (segment (start 149.67 91.5) (end 157.75 83.42) (width 0.2) (layer "B.Cu") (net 7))
 (segment (start 130.719662 89.446246) (end 130.691726 89.37776) (width 0.2) (layer "B.Cu") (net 1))
 (segment (start 156.599 74.411) (end 157.75 73.26) (width 0.2) (layer "B.Cu") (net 1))
 (segment (start 158.83776 73.26) (end 157.75 73.26) (width 0.2) (layer "B.Cu") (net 1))
 (segment (start 130.53125 83.32875) (end 139.449 74.411) (width 0.2) (layer "B.Cu") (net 1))
 (segment (start 130.53125 89.634658) (end 130.53125 83.32875) (width 0.2) (layer "B.Cu") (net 1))
 (segment (start 164.087501 78.509741) (end 158.83776 73.26) (width 0.2) (layer "B.Cu") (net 1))
 (segment (start 130.53125 89.634658) (end 130.719662 89.446246) (width 0.2) (layer "B.Cu") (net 1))
 (segment (start 139.449 74.411) (end 156.599 74.411) (width 0.2) (layer "B.Cu") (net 1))
 (segment (start 164.087501 89.634658) (end 164.087501 78.509741) (width 0.2) (layer "B.Cu") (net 1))
 (segment (start 147 81.02424) (end 142.92676 76.951) (width 0.2) (layer "F.Cu") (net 8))
 (segment (start 141.46224 73.26) (end 142.5 73.26) (width 0.2) (layer "F.Cu") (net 8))
 (segment (start 139.399 75.32324) (end 141.46224 73.26) (width 0.2) (layer "F.Cu") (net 8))
 (segment (start 139.399 76.27676) (end 139.399 75.32324) (width 0.2) (layer "F.Cu") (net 8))
 (segment (start 142.92676 76.951) (end 140.07324 76.951) (width 0.2) (layer "F.Cu") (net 8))
 (segment (start 147 97.7925) (end 147 81.02424) (width 0.2) (layer "F.Cu") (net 8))
 (segment (start 140.07324 76.951) (end 139.399 76.27676) (width 0.2) (layer "F.Cu") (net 8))
 (segment (start 142.71625 102.07625) (end 147 97.7925) (width 0.2) (layer "F.Cu") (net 8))
 (segment (start 142.5 75.8) (end 162.08375 95.38375) (width 0.2) (layer "F.Cu") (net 6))
 (segment (start 162.08375 95.38375) (end 162.08375 102.07625) (width 0.2) (layer "F.Cu") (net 6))
 (segment (start 128.5875 83.4125) (end 133.66 78.34) (width 0.2) (layer "F.Cu") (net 5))
 (segment (start 133.66 78.34) (end 142.5 78.34) (width 0.2) (layer "F.Cu") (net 5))
 (segment (start 142.875 121.44375) (end 142.875 128.5875) (width 0.2) (layer "F.Cu") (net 5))
 (segment (start 135.90753 128.87475) (end 128.5875 121.55472) (width 0.2) (layer "F.Cu") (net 5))
 (segment (start 142.875 128.5875) (end 142.58775 128.87475) (width 0.2) (layer "F.Cu") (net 5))
 (segment (start 128.5875 121.55472) (end 128.5875 83.4125) (width 0.2) (layer "F.Cu") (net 5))
 (segment (start 142.58775 128.87475) (end 135.90753 128.87475) (width 0.2) (layer "F.Cu") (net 5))
 (segment (start 135.944686 125.38475) (end 133.89525 123.335314) (width 0.2) (layer "F.Cu") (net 9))
 (segment (start 143.851 82.231) (end 142.5 80.88) (width 0.2) (layer "F.Cu") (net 9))
 (segment (start 163.5125 121.285) (end 161.956866 121.285) (width 0.2) (layer "F.Cu") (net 9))
 (segment (start 158.015866 125.226) (end 156.582186 125.226) (width 0.2) (layer "F.Cu") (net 9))
 (segment (start 148.438436 117.08225) (end 144.85525 117.08225) (width 0.2) (layer "F.Cu") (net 9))
 (segment (start 156.582186 125.226) (end 148.438436 117.08225) (width 0.2) (layer "F.Cu") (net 9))
 (segment (start 143.851 95.150186) (end 143.851 82.231) (width 0.2) (layer "F.Cu") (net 9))
 (segment (start 137.105314 125.38475) (end 135.944686 125.38475) (width 0.2) (layer "F.Cu") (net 9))
 (segment (start 161.956866 121.285) (end 158.015866 125.226) (width 0.2) (layer "F.Cu") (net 9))
 (segment (start 133.89525 123.335314) (end 133.89525 105.105936) (width 0.2) (layer "F.Cu") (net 9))
 (segment (start 138.5135 123.424) (end 138.5135 123.976564) (width 0.2) (layer "F.Cu") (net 9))
 (segment (start 144.85525 117.08225) (end 138.5135 123.424) (width 0.2) (layer "F.Cu") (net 9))
 (segment (start 138.5135 123.976564) (end 137.105314 125.38475) (width 0.2) (layer "F.Cu") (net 9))
 (segment (start 133.89525 105.105936) (end 143.851 95.150186) (width 0.2) (layer "F.Cu") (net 9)))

